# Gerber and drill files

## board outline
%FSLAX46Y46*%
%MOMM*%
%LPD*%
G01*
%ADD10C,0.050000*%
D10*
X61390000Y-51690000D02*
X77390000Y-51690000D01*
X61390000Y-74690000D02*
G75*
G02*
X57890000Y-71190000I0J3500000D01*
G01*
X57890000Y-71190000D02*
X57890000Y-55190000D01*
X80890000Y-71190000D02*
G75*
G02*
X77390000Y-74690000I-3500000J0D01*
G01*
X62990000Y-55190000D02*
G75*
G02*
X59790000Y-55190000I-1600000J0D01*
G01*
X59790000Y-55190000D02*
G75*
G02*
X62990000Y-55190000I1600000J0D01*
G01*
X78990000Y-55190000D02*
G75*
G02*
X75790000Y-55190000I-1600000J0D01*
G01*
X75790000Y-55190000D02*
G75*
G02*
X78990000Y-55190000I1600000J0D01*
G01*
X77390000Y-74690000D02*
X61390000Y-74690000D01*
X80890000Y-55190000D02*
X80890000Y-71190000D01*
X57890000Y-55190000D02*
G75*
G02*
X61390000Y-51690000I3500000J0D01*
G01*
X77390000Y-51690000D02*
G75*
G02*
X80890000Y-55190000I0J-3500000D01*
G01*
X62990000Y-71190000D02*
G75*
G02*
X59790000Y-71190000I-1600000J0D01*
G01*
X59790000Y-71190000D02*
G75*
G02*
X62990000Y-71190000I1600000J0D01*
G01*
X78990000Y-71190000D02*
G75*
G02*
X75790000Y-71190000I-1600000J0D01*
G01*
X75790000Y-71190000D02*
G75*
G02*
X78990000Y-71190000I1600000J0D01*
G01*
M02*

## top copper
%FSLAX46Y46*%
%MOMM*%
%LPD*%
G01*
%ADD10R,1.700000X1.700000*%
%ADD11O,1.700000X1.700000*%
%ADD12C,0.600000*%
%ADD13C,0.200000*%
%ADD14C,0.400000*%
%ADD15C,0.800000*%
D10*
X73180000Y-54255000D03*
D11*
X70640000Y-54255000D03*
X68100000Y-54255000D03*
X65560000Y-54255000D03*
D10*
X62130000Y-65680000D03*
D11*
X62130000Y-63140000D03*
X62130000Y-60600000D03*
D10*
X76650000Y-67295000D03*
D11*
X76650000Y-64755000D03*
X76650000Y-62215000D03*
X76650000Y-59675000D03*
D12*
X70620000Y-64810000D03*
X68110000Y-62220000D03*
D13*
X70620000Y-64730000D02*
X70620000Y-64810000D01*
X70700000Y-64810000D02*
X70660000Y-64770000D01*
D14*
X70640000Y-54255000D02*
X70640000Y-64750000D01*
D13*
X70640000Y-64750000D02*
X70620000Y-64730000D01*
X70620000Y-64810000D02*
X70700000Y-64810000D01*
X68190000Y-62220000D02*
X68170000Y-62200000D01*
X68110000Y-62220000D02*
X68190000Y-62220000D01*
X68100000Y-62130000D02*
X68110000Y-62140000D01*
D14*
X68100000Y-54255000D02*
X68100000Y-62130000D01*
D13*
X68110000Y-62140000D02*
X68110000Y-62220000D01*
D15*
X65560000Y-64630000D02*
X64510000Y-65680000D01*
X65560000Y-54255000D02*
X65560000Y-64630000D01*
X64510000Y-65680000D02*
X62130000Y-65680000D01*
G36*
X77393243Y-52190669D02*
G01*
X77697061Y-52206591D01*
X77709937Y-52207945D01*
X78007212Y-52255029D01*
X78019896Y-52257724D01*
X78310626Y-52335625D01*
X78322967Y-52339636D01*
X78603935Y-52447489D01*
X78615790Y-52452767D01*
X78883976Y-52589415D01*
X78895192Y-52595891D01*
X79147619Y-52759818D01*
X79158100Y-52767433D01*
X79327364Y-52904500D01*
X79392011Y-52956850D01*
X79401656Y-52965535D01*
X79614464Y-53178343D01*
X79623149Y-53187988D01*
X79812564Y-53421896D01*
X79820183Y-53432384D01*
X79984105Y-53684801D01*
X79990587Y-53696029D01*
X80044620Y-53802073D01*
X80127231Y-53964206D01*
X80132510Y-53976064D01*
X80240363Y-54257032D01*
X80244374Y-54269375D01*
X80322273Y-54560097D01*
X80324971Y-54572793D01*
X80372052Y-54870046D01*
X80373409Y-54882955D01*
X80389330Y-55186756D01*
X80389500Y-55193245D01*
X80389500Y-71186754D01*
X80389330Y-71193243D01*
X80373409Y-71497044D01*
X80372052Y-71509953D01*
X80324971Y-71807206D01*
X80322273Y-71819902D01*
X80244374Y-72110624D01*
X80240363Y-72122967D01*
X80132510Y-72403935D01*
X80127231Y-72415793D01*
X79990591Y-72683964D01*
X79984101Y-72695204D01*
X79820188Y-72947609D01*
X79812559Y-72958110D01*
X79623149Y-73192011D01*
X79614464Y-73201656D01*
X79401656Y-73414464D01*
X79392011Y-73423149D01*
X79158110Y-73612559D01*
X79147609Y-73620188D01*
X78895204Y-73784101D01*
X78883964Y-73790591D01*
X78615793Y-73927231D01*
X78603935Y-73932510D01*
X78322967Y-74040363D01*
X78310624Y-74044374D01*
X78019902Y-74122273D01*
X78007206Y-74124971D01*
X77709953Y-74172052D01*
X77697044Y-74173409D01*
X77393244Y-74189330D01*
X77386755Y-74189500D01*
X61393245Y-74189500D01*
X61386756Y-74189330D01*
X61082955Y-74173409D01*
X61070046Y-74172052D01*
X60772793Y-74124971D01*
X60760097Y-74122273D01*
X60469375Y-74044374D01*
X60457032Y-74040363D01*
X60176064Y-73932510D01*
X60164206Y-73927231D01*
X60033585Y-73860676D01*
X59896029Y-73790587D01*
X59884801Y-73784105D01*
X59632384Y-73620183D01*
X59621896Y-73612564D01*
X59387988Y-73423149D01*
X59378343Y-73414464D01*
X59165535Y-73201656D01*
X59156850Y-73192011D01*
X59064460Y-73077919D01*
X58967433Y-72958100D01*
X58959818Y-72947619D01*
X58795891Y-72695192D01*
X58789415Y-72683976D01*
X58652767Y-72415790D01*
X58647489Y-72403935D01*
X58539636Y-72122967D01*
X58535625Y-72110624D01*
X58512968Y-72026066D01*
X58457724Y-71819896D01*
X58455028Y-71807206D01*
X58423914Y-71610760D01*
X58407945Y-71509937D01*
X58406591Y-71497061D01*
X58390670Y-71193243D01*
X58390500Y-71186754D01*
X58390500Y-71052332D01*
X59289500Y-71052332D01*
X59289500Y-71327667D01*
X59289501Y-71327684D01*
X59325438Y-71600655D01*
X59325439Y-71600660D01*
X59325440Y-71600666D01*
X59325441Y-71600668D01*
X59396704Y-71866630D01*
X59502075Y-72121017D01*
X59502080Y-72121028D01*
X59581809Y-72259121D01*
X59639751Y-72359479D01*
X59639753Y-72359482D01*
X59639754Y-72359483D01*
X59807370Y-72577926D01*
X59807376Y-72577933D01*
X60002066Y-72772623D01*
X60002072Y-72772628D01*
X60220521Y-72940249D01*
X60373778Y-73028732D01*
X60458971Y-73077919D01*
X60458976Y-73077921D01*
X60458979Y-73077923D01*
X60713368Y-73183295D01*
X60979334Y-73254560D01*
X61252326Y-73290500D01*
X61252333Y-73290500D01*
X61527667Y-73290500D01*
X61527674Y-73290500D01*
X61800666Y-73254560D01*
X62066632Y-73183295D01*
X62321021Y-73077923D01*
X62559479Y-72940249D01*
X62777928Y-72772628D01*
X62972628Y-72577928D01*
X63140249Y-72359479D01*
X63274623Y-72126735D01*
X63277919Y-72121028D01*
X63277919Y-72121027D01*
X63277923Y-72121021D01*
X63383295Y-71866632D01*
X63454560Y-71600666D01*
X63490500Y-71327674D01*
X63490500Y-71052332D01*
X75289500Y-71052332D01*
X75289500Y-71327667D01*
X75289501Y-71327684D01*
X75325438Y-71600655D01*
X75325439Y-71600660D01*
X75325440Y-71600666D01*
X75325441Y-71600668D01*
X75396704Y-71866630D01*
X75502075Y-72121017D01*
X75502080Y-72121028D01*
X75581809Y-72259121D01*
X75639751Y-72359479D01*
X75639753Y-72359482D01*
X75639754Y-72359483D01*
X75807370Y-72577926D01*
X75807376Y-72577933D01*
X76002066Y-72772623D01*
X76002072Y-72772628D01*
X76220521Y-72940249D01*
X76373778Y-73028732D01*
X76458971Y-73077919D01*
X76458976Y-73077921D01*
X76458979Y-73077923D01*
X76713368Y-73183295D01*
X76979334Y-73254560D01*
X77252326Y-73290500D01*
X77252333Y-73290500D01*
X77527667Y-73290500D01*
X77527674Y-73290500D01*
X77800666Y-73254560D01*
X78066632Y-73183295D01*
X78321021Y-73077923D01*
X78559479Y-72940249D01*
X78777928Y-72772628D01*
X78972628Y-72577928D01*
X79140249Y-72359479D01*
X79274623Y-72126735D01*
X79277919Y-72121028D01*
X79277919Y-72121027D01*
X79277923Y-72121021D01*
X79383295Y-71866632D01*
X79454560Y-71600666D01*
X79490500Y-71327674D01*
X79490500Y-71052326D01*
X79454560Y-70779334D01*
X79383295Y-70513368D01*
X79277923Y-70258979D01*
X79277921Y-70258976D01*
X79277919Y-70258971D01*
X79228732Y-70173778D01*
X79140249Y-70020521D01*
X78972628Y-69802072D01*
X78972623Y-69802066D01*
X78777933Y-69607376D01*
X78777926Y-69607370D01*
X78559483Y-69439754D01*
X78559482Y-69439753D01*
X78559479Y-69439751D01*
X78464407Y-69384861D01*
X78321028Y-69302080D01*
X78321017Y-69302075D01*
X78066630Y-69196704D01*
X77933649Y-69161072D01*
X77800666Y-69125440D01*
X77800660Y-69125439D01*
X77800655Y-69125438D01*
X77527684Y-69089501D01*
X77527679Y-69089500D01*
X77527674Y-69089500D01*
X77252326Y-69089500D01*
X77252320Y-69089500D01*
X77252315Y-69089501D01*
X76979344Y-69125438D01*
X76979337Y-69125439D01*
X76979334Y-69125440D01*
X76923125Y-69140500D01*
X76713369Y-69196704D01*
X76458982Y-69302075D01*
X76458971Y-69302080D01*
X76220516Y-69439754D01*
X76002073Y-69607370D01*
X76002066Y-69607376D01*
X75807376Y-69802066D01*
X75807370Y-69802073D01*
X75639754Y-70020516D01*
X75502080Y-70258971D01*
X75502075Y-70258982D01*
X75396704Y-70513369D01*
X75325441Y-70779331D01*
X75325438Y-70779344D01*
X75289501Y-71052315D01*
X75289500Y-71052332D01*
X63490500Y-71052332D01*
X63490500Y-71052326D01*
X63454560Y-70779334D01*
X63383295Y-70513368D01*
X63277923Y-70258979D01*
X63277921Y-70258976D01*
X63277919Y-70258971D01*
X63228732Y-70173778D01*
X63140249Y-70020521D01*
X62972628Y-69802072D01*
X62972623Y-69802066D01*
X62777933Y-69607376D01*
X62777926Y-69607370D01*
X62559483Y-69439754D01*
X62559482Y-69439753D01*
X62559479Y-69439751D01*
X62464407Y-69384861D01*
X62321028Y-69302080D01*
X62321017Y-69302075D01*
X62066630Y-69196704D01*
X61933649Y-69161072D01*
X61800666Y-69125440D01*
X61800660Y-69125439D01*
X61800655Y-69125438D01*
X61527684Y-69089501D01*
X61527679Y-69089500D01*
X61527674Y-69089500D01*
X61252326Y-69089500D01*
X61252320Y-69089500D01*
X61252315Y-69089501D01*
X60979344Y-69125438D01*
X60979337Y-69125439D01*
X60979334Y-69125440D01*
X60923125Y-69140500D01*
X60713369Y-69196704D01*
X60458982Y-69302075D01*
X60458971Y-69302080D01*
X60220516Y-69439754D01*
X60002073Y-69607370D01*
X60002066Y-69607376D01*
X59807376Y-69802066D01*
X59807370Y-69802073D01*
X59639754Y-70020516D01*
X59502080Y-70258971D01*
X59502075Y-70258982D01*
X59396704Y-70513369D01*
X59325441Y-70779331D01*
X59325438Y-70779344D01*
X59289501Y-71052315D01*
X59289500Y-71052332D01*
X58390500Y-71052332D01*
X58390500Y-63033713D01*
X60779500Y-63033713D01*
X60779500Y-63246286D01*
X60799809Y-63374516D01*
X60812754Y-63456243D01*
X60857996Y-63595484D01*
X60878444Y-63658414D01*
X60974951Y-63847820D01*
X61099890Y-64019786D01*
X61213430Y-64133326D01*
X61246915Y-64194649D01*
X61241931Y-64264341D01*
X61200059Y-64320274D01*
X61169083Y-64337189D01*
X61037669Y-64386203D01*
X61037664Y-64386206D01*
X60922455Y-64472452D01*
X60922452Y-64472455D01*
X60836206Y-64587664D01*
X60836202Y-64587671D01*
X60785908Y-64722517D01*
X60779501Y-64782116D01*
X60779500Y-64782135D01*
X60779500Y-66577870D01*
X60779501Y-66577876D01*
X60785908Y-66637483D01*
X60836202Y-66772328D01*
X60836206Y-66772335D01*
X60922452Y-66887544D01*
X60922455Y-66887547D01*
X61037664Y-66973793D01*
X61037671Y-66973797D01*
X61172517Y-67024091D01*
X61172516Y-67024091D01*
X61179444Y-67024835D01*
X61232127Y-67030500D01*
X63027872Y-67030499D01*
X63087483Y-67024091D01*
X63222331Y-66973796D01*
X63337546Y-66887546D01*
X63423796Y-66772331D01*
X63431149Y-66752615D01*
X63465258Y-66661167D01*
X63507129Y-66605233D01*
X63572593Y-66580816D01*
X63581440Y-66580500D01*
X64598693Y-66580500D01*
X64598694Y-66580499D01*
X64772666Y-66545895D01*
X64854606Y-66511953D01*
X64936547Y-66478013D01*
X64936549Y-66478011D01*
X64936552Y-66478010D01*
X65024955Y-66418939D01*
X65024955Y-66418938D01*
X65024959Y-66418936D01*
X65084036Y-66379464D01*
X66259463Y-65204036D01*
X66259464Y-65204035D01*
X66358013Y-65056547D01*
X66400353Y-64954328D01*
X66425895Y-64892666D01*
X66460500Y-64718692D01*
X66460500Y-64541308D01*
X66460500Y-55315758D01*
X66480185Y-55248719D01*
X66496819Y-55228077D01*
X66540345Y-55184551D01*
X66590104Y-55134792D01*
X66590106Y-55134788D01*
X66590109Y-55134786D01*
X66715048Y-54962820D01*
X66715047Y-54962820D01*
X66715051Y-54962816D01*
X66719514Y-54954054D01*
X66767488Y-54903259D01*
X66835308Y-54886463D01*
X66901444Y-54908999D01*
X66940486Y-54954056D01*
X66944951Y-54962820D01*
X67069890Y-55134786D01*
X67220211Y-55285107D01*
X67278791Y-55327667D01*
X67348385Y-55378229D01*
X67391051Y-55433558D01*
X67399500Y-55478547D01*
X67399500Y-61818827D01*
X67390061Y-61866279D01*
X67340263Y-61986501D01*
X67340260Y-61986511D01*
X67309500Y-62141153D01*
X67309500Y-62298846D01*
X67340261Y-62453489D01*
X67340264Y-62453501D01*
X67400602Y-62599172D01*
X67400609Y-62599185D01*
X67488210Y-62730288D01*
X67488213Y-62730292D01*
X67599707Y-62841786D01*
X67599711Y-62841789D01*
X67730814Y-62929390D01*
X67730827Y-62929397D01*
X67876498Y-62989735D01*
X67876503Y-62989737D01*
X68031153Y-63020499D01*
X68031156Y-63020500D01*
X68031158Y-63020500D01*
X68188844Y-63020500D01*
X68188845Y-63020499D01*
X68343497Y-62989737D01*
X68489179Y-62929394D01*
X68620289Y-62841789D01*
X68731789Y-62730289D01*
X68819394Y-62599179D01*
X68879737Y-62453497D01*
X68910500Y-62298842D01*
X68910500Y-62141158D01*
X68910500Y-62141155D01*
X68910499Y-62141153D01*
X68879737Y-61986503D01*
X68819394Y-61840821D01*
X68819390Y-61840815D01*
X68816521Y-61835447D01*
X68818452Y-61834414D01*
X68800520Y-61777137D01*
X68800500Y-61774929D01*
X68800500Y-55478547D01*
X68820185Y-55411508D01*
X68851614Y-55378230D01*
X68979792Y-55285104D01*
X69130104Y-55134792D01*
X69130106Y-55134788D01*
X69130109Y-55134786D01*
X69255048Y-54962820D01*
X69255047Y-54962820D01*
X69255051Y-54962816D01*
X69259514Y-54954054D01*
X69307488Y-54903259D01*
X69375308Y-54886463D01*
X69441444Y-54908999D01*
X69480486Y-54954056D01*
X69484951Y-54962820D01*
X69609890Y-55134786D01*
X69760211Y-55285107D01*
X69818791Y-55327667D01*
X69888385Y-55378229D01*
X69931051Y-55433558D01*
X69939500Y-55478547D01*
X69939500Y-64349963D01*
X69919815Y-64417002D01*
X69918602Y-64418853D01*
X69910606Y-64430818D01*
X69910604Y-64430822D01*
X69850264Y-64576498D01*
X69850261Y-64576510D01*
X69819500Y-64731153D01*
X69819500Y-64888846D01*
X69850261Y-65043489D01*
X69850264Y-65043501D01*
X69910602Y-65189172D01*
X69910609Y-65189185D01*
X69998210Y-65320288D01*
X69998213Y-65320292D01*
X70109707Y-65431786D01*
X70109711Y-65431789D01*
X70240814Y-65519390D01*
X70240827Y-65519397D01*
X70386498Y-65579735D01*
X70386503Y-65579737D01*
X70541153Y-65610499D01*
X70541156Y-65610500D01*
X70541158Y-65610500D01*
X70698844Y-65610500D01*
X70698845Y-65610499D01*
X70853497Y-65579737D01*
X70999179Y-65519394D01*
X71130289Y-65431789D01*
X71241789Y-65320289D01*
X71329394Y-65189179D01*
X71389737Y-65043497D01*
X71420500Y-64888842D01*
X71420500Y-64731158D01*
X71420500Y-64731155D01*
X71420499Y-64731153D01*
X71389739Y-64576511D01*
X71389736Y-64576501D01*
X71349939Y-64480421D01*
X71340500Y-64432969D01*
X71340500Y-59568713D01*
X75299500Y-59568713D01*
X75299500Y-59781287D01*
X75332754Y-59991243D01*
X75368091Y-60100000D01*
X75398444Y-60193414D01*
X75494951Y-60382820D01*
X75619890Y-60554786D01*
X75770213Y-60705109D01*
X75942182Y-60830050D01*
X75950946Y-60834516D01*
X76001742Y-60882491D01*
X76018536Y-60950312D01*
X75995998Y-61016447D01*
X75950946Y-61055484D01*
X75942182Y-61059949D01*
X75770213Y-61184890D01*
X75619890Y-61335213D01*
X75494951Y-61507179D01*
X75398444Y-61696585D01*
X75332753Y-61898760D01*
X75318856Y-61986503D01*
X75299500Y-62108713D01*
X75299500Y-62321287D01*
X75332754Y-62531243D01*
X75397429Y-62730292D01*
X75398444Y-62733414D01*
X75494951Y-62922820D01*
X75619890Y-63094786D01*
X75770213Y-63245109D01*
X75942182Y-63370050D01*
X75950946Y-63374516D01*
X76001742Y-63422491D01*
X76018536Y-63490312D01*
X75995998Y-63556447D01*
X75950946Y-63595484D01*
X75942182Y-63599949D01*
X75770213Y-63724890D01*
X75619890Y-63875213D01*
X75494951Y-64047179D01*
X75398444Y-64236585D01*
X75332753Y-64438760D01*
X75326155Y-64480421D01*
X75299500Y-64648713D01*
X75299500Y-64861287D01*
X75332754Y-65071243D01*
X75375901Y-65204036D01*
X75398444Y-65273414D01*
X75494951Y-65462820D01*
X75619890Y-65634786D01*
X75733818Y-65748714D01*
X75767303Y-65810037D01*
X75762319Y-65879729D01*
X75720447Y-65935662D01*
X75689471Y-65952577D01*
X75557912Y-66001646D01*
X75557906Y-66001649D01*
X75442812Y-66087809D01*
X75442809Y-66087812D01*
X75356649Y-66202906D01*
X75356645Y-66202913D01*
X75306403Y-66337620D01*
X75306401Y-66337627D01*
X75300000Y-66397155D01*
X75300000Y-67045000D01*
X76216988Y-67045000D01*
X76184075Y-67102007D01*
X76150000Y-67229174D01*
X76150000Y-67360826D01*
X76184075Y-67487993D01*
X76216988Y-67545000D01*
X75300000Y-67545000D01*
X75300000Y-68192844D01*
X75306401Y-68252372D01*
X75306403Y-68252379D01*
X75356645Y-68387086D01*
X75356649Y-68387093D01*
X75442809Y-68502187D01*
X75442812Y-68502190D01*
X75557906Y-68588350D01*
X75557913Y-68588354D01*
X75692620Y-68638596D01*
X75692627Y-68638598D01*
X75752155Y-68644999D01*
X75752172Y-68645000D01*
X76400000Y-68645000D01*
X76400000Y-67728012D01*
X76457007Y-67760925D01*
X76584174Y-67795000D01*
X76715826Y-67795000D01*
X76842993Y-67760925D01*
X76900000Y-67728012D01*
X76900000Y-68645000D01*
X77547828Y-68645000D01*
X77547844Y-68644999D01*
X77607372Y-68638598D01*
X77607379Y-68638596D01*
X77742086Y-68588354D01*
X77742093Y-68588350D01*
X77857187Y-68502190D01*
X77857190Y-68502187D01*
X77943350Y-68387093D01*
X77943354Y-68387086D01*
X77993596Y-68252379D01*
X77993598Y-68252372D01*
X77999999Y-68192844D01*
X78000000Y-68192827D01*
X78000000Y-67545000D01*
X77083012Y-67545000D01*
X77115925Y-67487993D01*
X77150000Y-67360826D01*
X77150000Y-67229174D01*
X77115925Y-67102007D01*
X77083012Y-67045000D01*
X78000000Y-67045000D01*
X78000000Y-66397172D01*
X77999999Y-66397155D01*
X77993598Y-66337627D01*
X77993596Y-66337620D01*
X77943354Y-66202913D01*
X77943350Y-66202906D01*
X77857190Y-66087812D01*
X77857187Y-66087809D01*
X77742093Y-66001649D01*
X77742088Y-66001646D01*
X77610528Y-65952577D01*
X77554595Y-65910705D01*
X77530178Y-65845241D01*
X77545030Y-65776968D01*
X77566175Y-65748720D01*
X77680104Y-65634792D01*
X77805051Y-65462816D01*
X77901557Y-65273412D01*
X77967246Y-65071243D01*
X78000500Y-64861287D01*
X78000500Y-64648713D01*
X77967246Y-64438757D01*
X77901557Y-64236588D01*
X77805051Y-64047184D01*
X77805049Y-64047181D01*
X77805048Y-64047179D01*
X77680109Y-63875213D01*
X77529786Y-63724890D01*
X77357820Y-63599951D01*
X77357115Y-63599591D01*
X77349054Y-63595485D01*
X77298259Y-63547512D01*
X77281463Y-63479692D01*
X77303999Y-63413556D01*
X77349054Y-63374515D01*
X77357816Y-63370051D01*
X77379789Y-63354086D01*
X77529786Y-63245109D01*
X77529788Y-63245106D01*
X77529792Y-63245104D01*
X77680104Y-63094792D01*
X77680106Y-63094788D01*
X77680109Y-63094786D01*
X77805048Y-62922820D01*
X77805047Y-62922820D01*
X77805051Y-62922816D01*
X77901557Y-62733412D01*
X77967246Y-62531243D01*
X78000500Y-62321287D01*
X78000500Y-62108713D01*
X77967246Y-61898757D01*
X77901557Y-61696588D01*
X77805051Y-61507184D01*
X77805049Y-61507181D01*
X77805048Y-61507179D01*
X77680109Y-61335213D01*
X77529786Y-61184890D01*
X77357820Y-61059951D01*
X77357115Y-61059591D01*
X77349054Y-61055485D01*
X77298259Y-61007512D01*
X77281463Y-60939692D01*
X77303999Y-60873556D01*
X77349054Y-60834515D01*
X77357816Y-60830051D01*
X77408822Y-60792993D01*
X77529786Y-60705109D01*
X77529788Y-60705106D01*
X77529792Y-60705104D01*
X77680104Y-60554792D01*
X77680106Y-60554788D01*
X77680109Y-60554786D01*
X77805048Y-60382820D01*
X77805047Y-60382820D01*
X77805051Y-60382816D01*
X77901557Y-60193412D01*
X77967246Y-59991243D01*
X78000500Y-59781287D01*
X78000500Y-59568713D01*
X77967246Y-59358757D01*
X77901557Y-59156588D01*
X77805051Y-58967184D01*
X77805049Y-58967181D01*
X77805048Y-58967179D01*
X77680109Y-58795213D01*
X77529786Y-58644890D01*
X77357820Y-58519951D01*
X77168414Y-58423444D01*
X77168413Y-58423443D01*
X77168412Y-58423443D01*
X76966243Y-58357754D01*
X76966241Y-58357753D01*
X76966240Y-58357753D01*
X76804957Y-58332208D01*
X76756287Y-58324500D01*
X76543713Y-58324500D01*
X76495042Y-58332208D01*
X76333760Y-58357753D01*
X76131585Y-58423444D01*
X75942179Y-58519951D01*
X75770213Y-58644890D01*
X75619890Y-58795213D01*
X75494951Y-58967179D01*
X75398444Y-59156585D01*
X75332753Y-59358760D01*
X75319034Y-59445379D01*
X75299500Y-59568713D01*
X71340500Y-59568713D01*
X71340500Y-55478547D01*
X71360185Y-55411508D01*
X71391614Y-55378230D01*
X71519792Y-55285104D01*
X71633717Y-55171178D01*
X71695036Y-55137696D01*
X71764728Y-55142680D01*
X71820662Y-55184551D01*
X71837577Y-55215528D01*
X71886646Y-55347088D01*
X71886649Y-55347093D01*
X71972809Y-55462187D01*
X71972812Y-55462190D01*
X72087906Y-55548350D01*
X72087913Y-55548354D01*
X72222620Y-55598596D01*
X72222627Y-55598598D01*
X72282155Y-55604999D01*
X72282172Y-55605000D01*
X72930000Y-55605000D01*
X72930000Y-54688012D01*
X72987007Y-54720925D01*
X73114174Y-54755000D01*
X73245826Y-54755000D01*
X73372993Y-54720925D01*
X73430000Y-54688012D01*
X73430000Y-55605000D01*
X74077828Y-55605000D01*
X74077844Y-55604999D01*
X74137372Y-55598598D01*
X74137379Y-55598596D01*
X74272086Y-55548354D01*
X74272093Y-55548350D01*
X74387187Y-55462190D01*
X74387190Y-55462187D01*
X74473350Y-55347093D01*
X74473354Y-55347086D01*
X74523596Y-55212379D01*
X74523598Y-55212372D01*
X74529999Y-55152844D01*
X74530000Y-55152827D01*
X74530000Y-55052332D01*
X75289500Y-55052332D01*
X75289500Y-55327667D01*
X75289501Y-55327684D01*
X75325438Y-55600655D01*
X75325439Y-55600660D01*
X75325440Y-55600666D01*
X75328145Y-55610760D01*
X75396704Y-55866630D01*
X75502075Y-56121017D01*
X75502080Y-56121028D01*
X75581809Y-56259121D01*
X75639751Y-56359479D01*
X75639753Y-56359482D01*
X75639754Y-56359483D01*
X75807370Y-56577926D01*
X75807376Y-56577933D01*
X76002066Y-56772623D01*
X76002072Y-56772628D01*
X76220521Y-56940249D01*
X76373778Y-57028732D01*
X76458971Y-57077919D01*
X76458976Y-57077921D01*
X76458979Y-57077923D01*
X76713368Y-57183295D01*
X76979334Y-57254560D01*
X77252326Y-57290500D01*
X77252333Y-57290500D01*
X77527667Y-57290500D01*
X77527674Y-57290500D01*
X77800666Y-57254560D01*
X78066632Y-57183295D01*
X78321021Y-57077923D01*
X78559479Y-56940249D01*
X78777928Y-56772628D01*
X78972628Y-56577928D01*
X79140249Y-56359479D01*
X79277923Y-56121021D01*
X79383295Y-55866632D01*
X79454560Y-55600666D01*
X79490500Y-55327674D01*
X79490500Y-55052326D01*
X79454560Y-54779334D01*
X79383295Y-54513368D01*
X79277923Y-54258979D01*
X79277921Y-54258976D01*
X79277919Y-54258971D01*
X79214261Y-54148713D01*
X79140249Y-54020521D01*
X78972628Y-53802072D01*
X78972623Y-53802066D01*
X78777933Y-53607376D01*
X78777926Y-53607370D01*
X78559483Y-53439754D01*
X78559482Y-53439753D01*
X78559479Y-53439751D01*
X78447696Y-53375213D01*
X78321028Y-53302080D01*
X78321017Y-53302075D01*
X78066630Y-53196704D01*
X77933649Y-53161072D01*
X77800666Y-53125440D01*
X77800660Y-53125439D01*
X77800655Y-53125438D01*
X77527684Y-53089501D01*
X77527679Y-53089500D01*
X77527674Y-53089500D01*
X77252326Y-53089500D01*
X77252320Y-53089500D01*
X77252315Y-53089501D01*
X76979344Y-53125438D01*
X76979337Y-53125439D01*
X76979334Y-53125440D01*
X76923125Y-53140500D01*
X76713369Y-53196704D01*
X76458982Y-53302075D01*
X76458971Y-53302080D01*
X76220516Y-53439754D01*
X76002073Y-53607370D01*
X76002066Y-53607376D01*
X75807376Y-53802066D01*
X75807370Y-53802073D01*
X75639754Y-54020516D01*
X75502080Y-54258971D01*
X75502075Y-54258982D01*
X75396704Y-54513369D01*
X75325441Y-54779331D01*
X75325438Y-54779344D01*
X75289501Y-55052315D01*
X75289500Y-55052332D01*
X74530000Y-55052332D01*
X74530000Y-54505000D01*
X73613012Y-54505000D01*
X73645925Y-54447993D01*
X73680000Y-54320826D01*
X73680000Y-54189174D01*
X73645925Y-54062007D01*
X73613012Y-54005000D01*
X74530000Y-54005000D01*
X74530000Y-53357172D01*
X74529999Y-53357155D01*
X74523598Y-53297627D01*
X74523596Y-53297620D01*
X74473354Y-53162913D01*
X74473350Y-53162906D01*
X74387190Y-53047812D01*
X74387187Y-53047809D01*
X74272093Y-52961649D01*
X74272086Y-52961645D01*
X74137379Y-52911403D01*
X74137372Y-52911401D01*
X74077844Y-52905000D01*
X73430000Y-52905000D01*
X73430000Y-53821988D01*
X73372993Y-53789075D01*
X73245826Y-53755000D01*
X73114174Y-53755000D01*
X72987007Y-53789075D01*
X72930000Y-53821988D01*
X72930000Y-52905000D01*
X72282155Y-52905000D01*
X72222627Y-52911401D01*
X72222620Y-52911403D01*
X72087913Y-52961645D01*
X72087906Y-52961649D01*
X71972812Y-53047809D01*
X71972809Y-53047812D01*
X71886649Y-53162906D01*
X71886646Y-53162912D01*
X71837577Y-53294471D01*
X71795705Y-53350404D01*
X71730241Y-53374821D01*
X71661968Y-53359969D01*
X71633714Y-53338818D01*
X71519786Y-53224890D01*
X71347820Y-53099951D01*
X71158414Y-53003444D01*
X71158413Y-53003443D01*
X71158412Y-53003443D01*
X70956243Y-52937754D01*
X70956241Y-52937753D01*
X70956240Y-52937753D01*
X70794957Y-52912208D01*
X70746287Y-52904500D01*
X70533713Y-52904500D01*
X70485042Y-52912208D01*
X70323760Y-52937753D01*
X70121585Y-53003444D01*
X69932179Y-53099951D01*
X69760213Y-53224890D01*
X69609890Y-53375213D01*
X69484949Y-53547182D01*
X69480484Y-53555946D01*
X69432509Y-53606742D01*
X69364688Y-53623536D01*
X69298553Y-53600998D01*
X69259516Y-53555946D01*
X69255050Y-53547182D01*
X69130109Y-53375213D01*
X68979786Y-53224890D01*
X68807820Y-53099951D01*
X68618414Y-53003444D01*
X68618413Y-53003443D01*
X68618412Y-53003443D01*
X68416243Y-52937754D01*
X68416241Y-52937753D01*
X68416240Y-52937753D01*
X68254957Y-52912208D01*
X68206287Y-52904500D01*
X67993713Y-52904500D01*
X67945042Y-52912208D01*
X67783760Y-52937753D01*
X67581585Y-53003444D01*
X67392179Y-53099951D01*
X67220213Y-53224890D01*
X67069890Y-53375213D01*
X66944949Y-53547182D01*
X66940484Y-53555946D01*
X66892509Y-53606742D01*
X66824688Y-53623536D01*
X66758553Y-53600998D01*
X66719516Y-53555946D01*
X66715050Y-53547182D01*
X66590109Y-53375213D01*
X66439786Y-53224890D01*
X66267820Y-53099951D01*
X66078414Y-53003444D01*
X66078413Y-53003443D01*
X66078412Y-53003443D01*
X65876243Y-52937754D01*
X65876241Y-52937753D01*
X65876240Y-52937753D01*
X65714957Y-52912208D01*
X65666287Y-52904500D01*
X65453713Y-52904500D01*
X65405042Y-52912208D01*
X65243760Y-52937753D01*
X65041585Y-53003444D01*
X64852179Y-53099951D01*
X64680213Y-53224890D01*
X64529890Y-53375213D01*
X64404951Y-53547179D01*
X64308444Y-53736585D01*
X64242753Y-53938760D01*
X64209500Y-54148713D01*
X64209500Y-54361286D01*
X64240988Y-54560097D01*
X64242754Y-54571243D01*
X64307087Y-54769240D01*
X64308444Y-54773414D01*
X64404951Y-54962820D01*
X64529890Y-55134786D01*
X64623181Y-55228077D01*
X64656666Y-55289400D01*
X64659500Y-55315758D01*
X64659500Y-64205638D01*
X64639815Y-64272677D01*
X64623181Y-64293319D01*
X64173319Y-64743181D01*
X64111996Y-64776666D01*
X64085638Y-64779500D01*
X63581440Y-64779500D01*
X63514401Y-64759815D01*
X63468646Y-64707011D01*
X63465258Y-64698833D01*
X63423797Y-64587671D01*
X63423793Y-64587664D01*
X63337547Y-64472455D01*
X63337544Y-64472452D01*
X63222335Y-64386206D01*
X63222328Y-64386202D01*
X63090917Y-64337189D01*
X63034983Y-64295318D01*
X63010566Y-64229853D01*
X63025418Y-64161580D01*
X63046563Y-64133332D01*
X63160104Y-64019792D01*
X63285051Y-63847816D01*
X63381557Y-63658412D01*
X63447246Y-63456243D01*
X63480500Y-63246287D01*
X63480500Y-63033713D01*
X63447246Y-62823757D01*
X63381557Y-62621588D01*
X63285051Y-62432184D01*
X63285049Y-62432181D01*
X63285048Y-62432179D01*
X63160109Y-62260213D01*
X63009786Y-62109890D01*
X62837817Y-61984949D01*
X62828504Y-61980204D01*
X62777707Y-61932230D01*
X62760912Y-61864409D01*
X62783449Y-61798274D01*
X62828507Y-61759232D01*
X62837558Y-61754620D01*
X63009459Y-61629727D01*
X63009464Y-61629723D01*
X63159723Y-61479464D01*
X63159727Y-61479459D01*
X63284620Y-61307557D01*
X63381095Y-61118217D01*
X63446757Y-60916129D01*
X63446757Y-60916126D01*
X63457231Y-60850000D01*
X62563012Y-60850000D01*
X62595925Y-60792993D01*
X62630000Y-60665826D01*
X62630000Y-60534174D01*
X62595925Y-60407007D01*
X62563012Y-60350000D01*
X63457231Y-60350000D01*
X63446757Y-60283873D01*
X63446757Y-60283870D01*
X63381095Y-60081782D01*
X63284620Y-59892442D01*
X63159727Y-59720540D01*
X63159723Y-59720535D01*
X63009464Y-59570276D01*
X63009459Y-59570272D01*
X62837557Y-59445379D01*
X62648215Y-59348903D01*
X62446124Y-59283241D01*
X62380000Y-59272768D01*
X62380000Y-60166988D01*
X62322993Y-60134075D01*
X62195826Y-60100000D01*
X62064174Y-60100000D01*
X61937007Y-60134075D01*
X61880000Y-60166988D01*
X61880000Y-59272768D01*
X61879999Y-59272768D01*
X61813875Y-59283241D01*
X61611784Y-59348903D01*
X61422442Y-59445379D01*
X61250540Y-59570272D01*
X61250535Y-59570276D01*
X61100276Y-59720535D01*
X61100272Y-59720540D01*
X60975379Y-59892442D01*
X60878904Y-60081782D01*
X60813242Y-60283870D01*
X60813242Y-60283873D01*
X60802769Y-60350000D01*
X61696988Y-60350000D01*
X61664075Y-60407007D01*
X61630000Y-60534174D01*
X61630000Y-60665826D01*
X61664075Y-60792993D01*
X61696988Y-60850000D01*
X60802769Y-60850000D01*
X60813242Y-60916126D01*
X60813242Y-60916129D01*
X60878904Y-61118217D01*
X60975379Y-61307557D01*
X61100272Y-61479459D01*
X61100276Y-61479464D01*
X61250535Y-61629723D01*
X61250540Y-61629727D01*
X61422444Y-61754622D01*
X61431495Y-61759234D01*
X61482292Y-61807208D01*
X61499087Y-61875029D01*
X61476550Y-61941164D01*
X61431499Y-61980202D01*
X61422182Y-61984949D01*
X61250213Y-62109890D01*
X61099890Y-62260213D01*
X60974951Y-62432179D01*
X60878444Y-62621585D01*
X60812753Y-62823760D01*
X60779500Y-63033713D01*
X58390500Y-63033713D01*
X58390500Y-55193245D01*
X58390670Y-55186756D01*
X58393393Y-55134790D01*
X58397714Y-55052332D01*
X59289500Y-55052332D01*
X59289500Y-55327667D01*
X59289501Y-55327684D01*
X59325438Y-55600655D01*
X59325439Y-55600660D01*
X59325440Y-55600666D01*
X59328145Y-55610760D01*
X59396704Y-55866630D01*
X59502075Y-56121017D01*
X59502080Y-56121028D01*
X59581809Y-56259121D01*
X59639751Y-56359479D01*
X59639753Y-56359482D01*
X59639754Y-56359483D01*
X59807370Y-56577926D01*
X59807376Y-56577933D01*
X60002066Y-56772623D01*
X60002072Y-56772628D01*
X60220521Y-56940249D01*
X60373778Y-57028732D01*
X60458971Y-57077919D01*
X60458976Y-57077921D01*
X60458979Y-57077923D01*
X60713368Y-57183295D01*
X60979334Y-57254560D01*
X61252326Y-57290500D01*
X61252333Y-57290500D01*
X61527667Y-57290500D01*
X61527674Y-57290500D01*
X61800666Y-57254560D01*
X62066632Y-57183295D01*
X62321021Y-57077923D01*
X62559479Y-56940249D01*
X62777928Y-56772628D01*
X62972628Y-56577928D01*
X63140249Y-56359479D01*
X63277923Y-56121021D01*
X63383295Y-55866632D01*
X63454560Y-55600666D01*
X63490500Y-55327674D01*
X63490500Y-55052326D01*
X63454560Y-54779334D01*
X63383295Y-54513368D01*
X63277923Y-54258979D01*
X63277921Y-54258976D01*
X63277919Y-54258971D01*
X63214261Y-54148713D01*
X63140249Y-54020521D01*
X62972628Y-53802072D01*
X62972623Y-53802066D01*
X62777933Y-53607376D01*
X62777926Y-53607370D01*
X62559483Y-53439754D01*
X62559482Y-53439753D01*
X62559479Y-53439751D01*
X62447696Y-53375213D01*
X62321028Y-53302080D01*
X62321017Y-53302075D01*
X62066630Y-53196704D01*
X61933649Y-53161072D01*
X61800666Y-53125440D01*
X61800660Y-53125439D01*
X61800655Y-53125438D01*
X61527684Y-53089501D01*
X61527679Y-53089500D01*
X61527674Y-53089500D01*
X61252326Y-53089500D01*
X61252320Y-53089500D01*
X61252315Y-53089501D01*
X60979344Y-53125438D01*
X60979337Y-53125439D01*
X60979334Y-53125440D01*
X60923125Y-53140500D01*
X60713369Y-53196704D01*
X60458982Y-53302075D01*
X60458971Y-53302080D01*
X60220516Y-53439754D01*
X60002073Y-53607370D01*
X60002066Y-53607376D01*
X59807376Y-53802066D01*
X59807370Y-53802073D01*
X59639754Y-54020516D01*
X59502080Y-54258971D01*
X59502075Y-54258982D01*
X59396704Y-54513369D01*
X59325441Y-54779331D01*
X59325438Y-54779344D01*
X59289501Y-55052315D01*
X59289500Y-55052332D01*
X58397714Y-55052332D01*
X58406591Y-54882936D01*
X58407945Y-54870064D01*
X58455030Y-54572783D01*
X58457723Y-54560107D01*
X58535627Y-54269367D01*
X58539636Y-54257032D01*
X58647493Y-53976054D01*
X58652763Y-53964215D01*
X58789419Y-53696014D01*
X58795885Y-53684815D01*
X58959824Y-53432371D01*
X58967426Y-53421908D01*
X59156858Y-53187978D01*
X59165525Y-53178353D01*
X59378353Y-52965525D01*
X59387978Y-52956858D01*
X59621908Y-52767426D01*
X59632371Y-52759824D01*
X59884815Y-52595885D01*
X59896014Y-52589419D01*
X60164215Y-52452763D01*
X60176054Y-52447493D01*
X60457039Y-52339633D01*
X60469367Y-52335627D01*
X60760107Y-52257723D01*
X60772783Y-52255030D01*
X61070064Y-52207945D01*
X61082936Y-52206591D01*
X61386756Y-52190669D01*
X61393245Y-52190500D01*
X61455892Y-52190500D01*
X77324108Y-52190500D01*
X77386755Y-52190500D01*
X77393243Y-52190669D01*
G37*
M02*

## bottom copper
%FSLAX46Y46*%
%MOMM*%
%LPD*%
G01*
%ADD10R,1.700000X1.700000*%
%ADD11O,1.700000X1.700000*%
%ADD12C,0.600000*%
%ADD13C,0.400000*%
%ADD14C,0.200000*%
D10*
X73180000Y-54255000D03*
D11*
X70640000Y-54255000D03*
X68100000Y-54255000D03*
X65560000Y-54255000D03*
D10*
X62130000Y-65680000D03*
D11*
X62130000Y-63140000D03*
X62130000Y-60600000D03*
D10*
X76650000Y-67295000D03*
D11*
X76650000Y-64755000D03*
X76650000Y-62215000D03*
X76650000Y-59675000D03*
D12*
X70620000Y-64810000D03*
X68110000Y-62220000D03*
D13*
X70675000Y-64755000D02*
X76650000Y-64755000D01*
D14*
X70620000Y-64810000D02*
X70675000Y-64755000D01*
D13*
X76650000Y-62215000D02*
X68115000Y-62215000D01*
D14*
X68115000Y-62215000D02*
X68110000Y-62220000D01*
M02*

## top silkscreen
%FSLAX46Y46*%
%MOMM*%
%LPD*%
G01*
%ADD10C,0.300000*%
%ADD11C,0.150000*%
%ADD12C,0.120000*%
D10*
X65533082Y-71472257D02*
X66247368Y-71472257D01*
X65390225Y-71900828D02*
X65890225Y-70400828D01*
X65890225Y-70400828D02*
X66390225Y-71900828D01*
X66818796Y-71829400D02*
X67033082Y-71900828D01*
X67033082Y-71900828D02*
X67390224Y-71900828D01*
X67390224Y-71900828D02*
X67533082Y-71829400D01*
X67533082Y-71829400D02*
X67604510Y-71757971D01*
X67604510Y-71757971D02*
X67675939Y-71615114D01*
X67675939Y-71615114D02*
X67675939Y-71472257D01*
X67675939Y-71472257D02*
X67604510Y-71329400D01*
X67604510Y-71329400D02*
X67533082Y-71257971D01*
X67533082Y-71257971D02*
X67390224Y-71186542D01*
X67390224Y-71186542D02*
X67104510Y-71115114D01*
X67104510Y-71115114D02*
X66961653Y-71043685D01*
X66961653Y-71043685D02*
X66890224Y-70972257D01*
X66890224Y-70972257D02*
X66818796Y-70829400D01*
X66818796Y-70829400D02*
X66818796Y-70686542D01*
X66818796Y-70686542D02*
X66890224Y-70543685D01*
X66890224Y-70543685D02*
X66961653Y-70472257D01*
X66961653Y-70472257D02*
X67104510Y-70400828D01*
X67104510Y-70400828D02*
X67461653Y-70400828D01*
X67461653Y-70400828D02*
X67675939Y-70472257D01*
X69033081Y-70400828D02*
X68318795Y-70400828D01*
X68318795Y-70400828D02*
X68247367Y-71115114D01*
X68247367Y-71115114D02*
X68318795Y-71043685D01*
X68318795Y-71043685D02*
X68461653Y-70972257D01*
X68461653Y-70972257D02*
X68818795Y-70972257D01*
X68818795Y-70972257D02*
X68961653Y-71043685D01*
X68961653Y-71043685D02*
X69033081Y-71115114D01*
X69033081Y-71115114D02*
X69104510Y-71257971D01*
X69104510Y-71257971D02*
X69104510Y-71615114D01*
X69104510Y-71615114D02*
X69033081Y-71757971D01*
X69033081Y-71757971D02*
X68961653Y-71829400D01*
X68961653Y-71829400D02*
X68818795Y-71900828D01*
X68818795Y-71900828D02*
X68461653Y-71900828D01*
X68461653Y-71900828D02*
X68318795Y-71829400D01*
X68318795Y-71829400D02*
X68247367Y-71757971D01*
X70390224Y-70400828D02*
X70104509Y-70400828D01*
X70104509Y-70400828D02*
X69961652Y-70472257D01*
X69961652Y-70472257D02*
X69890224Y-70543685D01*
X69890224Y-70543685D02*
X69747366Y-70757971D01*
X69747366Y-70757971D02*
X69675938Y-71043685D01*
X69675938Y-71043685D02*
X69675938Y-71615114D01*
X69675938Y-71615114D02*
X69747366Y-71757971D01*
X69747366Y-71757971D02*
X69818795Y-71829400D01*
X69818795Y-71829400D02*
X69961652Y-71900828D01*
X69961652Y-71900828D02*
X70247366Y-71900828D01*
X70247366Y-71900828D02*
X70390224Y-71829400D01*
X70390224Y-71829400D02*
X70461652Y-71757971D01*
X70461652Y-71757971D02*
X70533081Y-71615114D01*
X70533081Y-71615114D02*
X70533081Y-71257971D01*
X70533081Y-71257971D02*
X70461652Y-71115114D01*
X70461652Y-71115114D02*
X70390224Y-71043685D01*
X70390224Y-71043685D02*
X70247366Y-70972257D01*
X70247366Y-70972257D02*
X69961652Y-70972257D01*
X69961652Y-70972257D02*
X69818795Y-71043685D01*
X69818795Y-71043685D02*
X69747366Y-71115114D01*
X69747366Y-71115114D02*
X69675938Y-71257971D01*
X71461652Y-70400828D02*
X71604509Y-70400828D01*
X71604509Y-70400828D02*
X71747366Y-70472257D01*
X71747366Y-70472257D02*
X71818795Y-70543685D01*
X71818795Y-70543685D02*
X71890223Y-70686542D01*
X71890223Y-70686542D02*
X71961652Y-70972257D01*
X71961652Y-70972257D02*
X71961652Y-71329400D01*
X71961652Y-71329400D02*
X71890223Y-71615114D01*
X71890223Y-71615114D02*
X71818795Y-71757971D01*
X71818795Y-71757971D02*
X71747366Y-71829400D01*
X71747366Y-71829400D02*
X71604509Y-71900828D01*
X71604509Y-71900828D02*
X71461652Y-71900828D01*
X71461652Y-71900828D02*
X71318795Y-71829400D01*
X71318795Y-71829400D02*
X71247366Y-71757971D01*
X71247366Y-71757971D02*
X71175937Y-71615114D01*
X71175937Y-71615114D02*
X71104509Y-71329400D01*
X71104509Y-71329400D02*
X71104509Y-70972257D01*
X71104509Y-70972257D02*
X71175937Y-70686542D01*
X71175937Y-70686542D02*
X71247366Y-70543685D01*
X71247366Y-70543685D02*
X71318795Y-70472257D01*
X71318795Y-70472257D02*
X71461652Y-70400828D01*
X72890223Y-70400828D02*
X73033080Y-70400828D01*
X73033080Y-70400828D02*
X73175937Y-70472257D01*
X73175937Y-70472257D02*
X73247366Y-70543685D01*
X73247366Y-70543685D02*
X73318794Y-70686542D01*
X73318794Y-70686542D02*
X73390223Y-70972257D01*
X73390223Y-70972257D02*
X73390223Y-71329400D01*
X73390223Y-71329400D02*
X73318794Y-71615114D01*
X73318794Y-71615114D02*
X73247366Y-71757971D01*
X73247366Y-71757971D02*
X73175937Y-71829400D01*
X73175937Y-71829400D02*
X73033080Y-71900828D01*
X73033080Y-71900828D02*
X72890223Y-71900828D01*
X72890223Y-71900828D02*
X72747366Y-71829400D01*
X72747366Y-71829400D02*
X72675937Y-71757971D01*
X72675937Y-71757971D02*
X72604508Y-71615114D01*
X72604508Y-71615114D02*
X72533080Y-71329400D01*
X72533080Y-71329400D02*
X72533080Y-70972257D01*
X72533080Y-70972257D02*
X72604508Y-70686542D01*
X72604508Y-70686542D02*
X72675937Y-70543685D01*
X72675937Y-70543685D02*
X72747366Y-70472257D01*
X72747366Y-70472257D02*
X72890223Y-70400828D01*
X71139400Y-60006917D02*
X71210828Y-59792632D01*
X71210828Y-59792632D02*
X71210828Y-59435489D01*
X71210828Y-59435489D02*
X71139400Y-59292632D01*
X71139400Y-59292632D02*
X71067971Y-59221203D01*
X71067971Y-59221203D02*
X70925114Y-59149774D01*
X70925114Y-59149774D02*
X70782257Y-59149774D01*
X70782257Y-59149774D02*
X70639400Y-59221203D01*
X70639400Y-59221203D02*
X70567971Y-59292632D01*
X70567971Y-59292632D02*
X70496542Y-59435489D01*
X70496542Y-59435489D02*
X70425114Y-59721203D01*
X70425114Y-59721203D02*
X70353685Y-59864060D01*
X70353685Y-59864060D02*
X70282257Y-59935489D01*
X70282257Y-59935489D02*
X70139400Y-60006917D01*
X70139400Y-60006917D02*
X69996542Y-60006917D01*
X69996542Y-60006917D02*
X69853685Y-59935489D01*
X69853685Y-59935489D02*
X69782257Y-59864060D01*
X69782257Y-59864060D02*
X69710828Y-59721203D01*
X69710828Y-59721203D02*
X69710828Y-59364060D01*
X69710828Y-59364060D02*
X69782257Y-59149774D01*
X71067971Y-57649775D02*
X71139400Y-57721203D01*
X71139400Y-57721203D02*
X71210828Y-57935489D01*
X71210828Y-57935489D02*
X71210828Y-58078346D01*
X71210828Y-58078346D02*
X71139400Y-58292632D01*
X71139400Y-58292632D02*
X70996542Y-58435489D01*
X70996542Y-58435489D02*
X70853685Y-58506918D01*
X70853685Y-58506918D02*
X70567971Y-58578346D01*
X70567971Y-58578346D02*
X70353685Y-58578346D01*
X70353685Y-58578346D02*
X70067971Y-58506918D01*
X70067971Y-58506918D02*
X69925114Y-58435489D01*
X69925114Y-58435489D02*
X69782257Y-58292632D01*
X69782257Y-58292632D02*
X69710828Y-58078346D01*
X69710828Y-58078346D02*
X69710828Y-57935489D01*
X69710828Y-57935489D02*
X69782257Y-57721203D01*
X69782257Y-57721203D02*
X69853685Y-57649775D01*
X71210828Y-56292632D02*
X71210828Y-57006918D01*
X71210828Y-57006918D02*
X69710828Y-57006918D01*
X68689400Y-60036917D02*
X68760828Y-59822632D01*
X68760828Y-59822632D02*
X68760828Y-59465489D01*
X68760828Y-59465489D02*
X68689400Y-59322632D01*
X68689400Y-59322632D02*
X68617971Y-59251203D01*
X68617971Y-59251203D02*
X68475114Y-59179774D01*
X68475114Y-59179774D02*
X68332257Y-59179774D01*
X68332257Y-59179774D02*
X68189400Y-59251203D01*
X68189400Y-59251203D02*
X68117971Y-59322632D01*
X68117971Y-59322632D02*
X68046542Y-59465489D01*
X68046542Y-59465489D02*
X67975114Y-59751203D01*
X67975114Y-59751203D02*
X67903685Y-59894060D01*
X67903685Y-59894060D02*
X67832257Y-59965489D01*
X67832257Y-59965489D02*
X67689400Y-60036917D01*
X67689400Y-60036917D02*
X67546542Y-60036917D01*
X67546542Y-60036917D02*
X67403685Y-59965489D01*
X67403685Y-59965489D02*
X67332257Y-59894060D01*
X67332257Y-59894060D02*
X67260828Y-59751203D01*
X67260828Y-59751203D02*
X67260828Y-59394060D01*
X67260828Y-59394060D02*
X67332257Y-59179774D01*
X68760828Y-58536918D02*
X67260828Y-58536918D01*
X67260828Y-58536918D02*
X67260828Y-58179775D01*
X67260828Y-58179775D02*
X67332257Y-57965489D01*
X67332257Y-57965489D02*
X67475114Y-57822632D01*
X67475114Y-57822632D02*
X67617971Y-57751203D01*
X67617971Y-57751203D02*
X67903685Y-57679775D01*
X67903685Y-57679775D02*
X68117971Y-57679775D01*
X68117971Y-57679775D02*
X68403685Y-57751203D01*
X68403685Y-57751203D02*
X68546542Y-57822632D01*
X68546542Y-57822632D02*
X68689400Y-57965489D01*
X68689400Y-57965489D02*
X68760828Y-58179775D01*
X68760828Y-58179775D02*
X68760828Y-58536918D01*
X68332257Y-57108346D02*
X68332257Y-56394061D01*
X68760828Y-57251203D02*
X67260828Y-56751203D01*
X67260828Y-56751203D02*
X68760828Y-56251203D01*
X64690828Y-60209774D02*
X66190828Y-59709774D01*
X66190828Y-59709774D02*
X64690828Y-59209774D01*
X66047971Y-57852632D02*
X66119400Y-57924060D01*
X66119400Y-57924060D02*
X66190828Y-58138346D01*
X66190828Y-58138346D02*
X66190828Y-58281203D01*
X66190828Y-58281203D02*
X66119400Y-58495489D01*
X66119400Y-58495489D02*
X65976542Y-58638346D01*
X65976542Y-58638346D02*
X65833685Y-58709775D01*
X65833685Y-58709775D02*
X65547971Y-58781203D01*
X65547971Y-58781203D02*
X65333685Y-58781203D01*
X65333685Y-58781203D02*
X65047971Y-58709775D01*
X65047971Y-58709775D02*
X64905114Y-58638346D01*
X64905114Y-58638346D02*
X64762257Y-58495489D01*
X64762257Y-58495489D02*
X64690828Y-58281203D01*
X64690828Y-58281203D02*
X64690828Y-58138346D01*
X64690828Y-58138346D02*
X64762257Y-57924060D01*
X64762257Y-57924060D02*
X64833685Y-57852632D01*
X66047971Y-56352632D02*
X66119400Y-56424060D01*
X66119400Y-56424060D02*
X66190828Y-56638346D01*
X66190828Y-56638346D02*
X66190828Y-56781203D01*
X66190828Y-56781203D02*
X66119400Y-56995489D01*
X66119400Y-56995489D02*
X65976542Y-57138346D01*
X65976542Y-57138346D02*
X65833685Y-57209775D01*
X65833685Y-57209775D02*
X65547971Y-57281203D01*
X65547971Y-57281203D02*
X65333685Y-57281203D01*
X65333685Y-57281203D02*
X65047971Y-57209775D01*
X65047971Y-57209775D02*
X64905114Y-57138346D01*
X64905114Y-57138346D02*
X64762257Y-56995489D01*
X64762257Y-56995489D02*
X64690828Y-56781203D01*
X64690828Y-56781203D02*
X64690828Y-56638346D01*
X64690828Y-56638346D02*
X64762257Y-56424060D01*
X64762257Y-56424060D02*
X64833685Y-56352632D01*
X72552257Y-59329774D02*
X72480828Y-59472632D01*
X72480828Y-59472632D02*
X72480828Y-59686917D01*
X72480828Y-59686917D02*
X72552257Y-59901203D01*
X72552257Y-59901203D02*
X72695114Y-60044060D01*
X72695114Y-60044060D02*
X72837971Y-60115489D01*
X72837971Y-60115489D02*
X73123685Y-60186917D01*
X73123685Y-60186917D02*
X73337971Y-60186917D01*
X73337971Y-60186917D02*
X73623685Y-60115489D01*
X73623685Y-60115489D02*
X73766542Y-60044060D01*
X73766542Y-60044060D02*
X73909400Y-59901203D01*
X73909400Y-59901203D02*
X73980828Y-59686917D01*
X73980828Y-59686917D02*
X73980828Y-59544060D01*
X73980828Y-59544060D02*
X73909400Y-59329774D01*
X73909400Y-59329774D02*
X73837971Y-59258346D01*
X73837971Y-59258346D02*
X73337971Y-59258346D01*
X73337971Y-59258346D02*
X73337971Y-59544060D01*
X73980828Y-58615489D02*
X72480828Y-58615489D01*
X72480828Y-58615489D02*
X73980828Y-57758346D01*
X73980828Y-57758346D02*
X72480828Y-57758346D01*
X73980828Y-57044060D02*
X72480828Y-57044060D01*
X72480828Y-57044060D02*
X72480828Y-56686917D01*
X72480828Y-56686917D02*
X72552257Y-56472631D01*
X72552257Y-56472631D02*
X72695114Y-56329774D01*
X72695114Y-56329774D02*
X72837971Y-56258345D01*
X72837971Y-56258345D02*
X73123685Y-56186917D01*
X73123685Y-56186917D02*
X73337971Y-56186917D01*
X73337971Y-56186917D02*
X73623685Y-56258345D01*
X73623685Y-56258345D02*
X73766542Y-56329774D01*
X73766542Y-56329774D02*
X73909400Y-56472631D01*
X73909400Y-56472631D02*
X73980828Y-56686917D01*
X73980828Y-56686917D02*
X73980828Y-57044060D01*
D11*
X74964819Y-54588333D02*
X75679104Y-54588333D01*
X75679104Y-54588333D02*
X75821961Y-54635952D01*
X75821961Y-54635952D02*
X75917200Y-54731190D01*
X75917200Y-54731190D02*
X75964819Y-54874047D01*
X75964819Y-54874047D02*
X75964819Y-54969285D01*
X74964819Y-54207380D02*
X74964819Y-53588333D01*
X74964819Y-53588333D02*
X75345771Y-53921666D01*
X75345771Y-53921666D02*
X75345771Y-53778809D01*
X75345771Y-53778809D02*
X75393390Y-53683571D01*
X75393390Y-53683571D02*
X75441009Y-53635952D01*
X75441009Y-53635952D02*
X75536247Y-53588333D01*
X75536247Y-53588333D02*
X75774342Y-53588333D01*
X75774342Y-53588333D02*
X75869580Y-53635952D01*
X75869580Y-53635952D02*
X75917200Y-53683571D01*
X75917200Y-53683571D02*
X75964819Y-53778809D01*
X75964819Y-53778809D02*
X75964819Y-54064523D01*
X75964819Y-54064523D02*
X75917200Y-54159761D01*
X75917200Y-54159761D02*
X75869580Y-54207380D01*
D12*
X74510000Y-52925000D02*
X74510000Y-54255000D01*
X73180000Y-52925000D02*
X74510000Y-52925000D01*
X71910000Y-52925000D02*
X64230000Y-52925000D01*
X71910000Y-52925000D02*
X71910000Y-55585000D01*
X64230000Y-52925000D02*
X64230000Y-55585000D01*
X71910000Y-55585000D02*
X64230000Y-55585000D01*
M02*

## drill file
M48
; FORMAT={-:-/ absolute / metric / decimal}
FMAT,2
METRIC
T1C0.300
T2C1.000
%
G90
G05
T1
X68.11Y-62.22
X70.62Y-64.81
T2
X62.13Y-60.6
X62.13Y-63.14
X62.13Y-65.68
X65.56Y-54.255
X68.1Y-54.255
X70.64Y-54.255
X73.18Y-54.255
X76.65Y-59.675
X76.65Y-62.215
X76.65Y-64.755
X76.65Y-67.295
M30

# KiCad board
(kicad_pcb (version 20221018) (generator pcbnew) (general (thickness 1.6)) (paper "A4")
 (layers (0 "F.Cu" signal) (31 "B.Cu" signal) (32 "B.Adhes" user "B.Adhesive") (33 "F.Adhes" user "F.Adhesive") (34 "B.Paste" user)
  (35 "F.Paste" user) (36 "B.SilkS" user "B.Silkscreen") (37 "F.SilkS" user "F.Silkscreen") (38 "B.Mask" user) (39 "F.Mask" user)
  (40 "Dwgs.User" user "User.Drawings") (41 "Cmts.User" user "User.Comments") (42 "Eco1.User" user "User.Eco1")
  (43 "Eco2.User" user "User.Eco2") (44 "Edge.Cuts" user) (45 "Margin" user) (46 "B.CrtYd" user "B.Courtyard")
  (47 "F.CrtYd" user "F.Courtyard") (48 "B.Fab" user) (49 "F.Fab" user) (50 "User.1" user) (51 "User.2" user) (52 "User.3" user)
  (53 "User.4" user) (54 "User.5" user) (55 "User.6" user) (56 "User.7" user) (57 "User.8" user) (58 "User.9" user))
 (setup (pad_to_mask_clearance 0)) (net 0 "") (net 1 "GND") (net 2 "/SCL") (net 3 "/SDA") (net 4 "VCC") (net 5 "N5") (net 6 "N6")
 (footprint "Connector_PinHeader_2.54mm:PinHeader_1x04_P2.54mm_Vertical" (layer "F.Cu") (at 73.18 54.255 -90)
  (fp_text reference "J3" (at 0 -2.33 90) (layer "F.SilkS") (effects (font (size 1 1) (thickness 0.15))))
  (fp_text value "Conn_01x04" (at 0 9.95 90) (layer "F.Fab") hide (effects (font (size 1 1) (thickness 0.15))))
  (fp_line (start -1.33 -1.33) (end 0 -1.33) (stroke (width 0.12) (type solid)) (layer "F.SilkS"))
  (fp_line (start -1.33 0) (end -1.33 -1.33) (stroke (width 0.12) (type solid)) (layer "F.SilkS"))
  (fp_line (start -1.33 1.27) (end -1.33 8.95) (stroke (width 0.12) (type solid)) (layer "F.SilkS"))
  (fp_line (start -1.33 1.27) (end 1.33 1.27) (stroke (width 0.12) (type solid)) (layer "F.SilkS"))
  (fp_line (start -1.33 8.95) (end 1.33 8.95) (stroke (width 0.12) (type solid)) (layer "F.SilkS"))
  (fp_line (start 1.33 1.27) (end 1.33 8.95) (stroke (width 0.12) (type solid)) (layer "F.SilkS"))
  (pad "1" thru_hole rect (at 0 0 270) (size 1.7 1.7) (drill 1) (layers "*.Cu" "*.Mask") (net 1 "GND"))
  (pad "2" thru_hole oval (at 0 2.54 270) (size 1.7 1.7) (drill 1) (layers "*.Cu" "*.Mask") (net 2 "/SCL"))
  (pad "3" thru_hole oval (at 0 5.08 270) (size 1.7 1.7) (drill 1) (layers "*.Cu" "*.Mask") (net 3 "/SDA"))
  (pad "4" thru_hole oval (at 0 7.62 270) (size 1.7 1.7) (drill 1) (layers "*.Cu" "*.Mask") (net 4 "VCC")))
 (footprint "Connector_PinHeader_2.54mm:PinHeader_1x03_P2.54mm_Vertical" (layer "B.Cu") (at 62.13 65.68)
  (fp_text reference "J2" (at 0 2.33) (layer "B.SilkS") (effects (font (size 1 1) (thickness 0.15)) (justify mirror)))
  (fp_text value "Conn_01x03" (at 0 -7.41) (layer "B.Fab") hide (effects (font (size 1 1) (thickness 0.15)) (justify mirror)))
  (pad "1" thru_hole rect (at 0 0) (size 1.7 1.7) (drill 1) (layers "*.Cu" "*.Mask") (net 4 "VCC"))
  (pad "2" thru_hole oval (at 0 -2.54) (size 1.7 1.7) (drill 1) (layers "*.Cu" "*.Mask") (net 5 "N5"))
  (pad "3" thru_hole oval (at 0 -5.08) (size 1.7 1.7) (drill 1) (layers "*.Cu" "*.Mask") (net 1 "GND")))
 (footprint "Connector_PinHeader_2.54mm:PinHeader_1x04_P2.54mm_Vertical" (layer "B.Cu") (at 76.65 67.295)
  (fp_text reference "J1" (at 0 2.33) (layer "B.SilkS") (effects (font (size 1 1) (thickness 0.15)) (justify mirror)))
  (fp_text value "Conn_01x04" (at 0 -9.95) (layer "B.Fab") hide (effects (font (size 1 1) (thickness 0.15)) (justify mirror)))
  (pad "1" thru_hole rect (at 0 0) (size 1.7 1.7) (drill 1) (layers "*.Cu" "*.Mask") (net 1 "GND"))
  (pad "2" thru_hole oval (at 0 -2.54) (size 1.7 1.7) (drill 1) (layers "*.Cu" "*.Mask") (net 2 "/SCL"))
  (pad "3" thru_hole oval (at 0 -5.08) (size 1.7 1.7) (drill 1) (layers "*.Cu" "*.Mask") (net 3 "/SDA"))
  (pad "4" thru_hole oval (at 0 -7.62) (size 1.7 1.7) (drill 1) (layers "*.Cu" "*.Mask") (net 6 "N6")))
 (gr_line (start 61.39 51.69) (end 77.39 51.69) (stroke (width 0.05) (type default)) (layer "Edge.Cuts"))
 (gr_arc (start 61.39 74.69) (mid 58.915126 73.664874) (end 57.89 71.19) (stroke (width 0.05) (type default)) (layer "Edge.Cuts"))
 (gr_line (start 57.89 71.19) (end 57.89 55.19) (stroke (width 0.05) (type default)) (layer "Edge.Cuts"))
 (gr_arc (start 80.89 71.19) (mid 79.864874 73.664874) (end 77.39 74.69) (stroke (width 0.05) (type default)) (layer "Edge.Cuts"))
 (gr_circle (center 61.39 55.19) (end 62.99 55.19) (stroke (width 0.05) (type default)) (fill none) (layer "Edge.Cuts"))
 (gr_circle (center 77.39 55.19) (end 78.99 55.19) (stroke (width 0.05) (type default)) (fill none) (layer "Edge.Cuts"))
 (gr_line (start 77.39 74.69) (end 61.39 74.69) (stroke (width 0.05) (type default)) (layer "Edge.Cuts"))
 (gr_line (start 80.89 55.19) (end 80.89 71.19) (stroke (width 0.05) (type default)) (layer "Edge.Cuts"))
 (gr_arc (start 57.89 55.19) (mid 58.915126 52.715126) (end 61.39 51.69) (stroke (width 0.05) (type default)) (layer "Edge.Cuts"))
 (gr_arc (start 77.39 51.69) (mid 79.864874 52.715126) (end 80.89 55.19) (stroke (width 0.05) (type default)) (layer "Edge.Cuts"))
 (gr_circle (center 61.39 71.19) (end 62.99 71.19) (stroke (width 0.05) (type default)) (fill none) (layer "Edge.Cuts"))
 (gr_circle (center 77.39 71.19) (end 78.99 71.19) (stroke (width 0.05) (type default)) (fill none) (layer "Edge.Cuts"))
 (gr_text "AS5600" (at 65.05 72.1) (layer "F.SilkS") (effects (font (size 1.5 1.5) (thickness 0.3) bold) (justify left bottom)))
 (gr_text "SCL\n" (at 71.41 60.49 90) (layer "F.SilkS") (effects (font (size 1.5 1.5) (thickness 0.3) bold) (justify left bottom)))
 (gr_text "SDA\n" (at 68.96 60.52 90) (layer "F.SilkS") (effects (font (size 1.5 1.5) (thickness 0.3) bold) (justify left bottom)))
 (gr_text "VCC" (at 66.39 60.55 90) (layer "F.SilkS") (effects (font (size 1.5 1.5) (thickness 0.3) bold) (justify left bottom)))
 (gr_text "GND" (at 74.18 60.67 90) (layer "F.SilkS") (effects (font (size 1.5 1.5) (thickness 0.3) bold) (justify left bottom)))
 (segment (start 70.62 64.73) (end 70.62 64.81) (width 0.2) (layer "F.Cu") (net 2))
 (segment (start 70.7 64.81) (end 70.66 64.77) (width 0.2) (layer "F.Cu") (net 2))
 (segment (start 70.64 54.255) (end 70.64 64.75) (width 0.4) (layer "F.Cu") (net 2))
 (segment (start 70.64 64.75) (end 70.62 64.73) (width 0.2) (layer "F.Cu") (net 2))
 (segment (start 70.62 64.81) (end 70.7 64.81) (width 0.2) (layer "F.Cu") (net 2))
 (via (at 70.62 64.81) (size 0.6) (drill 0.3) (layers "F.Cu" "B.Cu") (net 2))
 (segment (start 70.675 64.755) (end 76.65 64.755) (width 0.4) (layer "B.Cu") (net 2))
 (segment (start 70.62 64.81) (end 70.675 64.755) (width 0.2) (layer "B.Cu") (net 2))
 (segment (start 68.19 62.22) (end 68.17 62.2) (width 0.2) (layer "F.Cu") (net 3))
 (segment (start 68.11 62.22) (end 68.19 62.22) (width 0.2) (layer "F.Cu") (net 3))
 (segment (start 68.1 62.13) (end 68.11 62.14) (width 0.2) (layer "F.Cu") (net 3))
 (segment (start 68.1 54.255) (end 68.1 62.13) (width 0.4) (layer "F.Cu") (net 3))
 (segment (start 68.11 62.14) (end 68.11 62.22) (width 0.2) (layer "F.Cu") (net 3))
 (via (at 68.11 62.22) (size 0.6) (drill 0.3) (layers "F.Cu" "B.Cu") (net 3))
 (segment (start 76.65 62.215) (end 68.115 62.215) (width 0.4) (layer "B.Cu") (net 3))
 (segment (start 68.115 62.215) (end 68.11 62.22) (width 0.2) (layer "B.Cu") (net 3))
 (segment (start 65.56 64.63) (end 64.51 65.68) (width 0.8) (layer "F.Cu") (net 4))
 (segment (start 65.56 54.255) (end 65.56 64.63) (width 0.8) (layer "F.Cu") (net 4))
 (segment (start 64.51 65.68) (end 62.13 65.68) (width 0.8) (layer "F.Cu") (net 4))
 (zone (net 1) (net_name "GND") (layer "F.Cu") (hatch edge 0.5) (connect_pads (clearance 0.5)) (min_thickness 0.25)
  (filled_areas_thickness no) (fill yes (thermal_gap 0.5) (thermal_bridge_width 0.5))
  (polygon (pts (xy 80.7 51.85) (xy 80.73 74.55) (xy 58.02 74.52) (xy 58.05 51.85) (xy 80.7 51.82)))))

